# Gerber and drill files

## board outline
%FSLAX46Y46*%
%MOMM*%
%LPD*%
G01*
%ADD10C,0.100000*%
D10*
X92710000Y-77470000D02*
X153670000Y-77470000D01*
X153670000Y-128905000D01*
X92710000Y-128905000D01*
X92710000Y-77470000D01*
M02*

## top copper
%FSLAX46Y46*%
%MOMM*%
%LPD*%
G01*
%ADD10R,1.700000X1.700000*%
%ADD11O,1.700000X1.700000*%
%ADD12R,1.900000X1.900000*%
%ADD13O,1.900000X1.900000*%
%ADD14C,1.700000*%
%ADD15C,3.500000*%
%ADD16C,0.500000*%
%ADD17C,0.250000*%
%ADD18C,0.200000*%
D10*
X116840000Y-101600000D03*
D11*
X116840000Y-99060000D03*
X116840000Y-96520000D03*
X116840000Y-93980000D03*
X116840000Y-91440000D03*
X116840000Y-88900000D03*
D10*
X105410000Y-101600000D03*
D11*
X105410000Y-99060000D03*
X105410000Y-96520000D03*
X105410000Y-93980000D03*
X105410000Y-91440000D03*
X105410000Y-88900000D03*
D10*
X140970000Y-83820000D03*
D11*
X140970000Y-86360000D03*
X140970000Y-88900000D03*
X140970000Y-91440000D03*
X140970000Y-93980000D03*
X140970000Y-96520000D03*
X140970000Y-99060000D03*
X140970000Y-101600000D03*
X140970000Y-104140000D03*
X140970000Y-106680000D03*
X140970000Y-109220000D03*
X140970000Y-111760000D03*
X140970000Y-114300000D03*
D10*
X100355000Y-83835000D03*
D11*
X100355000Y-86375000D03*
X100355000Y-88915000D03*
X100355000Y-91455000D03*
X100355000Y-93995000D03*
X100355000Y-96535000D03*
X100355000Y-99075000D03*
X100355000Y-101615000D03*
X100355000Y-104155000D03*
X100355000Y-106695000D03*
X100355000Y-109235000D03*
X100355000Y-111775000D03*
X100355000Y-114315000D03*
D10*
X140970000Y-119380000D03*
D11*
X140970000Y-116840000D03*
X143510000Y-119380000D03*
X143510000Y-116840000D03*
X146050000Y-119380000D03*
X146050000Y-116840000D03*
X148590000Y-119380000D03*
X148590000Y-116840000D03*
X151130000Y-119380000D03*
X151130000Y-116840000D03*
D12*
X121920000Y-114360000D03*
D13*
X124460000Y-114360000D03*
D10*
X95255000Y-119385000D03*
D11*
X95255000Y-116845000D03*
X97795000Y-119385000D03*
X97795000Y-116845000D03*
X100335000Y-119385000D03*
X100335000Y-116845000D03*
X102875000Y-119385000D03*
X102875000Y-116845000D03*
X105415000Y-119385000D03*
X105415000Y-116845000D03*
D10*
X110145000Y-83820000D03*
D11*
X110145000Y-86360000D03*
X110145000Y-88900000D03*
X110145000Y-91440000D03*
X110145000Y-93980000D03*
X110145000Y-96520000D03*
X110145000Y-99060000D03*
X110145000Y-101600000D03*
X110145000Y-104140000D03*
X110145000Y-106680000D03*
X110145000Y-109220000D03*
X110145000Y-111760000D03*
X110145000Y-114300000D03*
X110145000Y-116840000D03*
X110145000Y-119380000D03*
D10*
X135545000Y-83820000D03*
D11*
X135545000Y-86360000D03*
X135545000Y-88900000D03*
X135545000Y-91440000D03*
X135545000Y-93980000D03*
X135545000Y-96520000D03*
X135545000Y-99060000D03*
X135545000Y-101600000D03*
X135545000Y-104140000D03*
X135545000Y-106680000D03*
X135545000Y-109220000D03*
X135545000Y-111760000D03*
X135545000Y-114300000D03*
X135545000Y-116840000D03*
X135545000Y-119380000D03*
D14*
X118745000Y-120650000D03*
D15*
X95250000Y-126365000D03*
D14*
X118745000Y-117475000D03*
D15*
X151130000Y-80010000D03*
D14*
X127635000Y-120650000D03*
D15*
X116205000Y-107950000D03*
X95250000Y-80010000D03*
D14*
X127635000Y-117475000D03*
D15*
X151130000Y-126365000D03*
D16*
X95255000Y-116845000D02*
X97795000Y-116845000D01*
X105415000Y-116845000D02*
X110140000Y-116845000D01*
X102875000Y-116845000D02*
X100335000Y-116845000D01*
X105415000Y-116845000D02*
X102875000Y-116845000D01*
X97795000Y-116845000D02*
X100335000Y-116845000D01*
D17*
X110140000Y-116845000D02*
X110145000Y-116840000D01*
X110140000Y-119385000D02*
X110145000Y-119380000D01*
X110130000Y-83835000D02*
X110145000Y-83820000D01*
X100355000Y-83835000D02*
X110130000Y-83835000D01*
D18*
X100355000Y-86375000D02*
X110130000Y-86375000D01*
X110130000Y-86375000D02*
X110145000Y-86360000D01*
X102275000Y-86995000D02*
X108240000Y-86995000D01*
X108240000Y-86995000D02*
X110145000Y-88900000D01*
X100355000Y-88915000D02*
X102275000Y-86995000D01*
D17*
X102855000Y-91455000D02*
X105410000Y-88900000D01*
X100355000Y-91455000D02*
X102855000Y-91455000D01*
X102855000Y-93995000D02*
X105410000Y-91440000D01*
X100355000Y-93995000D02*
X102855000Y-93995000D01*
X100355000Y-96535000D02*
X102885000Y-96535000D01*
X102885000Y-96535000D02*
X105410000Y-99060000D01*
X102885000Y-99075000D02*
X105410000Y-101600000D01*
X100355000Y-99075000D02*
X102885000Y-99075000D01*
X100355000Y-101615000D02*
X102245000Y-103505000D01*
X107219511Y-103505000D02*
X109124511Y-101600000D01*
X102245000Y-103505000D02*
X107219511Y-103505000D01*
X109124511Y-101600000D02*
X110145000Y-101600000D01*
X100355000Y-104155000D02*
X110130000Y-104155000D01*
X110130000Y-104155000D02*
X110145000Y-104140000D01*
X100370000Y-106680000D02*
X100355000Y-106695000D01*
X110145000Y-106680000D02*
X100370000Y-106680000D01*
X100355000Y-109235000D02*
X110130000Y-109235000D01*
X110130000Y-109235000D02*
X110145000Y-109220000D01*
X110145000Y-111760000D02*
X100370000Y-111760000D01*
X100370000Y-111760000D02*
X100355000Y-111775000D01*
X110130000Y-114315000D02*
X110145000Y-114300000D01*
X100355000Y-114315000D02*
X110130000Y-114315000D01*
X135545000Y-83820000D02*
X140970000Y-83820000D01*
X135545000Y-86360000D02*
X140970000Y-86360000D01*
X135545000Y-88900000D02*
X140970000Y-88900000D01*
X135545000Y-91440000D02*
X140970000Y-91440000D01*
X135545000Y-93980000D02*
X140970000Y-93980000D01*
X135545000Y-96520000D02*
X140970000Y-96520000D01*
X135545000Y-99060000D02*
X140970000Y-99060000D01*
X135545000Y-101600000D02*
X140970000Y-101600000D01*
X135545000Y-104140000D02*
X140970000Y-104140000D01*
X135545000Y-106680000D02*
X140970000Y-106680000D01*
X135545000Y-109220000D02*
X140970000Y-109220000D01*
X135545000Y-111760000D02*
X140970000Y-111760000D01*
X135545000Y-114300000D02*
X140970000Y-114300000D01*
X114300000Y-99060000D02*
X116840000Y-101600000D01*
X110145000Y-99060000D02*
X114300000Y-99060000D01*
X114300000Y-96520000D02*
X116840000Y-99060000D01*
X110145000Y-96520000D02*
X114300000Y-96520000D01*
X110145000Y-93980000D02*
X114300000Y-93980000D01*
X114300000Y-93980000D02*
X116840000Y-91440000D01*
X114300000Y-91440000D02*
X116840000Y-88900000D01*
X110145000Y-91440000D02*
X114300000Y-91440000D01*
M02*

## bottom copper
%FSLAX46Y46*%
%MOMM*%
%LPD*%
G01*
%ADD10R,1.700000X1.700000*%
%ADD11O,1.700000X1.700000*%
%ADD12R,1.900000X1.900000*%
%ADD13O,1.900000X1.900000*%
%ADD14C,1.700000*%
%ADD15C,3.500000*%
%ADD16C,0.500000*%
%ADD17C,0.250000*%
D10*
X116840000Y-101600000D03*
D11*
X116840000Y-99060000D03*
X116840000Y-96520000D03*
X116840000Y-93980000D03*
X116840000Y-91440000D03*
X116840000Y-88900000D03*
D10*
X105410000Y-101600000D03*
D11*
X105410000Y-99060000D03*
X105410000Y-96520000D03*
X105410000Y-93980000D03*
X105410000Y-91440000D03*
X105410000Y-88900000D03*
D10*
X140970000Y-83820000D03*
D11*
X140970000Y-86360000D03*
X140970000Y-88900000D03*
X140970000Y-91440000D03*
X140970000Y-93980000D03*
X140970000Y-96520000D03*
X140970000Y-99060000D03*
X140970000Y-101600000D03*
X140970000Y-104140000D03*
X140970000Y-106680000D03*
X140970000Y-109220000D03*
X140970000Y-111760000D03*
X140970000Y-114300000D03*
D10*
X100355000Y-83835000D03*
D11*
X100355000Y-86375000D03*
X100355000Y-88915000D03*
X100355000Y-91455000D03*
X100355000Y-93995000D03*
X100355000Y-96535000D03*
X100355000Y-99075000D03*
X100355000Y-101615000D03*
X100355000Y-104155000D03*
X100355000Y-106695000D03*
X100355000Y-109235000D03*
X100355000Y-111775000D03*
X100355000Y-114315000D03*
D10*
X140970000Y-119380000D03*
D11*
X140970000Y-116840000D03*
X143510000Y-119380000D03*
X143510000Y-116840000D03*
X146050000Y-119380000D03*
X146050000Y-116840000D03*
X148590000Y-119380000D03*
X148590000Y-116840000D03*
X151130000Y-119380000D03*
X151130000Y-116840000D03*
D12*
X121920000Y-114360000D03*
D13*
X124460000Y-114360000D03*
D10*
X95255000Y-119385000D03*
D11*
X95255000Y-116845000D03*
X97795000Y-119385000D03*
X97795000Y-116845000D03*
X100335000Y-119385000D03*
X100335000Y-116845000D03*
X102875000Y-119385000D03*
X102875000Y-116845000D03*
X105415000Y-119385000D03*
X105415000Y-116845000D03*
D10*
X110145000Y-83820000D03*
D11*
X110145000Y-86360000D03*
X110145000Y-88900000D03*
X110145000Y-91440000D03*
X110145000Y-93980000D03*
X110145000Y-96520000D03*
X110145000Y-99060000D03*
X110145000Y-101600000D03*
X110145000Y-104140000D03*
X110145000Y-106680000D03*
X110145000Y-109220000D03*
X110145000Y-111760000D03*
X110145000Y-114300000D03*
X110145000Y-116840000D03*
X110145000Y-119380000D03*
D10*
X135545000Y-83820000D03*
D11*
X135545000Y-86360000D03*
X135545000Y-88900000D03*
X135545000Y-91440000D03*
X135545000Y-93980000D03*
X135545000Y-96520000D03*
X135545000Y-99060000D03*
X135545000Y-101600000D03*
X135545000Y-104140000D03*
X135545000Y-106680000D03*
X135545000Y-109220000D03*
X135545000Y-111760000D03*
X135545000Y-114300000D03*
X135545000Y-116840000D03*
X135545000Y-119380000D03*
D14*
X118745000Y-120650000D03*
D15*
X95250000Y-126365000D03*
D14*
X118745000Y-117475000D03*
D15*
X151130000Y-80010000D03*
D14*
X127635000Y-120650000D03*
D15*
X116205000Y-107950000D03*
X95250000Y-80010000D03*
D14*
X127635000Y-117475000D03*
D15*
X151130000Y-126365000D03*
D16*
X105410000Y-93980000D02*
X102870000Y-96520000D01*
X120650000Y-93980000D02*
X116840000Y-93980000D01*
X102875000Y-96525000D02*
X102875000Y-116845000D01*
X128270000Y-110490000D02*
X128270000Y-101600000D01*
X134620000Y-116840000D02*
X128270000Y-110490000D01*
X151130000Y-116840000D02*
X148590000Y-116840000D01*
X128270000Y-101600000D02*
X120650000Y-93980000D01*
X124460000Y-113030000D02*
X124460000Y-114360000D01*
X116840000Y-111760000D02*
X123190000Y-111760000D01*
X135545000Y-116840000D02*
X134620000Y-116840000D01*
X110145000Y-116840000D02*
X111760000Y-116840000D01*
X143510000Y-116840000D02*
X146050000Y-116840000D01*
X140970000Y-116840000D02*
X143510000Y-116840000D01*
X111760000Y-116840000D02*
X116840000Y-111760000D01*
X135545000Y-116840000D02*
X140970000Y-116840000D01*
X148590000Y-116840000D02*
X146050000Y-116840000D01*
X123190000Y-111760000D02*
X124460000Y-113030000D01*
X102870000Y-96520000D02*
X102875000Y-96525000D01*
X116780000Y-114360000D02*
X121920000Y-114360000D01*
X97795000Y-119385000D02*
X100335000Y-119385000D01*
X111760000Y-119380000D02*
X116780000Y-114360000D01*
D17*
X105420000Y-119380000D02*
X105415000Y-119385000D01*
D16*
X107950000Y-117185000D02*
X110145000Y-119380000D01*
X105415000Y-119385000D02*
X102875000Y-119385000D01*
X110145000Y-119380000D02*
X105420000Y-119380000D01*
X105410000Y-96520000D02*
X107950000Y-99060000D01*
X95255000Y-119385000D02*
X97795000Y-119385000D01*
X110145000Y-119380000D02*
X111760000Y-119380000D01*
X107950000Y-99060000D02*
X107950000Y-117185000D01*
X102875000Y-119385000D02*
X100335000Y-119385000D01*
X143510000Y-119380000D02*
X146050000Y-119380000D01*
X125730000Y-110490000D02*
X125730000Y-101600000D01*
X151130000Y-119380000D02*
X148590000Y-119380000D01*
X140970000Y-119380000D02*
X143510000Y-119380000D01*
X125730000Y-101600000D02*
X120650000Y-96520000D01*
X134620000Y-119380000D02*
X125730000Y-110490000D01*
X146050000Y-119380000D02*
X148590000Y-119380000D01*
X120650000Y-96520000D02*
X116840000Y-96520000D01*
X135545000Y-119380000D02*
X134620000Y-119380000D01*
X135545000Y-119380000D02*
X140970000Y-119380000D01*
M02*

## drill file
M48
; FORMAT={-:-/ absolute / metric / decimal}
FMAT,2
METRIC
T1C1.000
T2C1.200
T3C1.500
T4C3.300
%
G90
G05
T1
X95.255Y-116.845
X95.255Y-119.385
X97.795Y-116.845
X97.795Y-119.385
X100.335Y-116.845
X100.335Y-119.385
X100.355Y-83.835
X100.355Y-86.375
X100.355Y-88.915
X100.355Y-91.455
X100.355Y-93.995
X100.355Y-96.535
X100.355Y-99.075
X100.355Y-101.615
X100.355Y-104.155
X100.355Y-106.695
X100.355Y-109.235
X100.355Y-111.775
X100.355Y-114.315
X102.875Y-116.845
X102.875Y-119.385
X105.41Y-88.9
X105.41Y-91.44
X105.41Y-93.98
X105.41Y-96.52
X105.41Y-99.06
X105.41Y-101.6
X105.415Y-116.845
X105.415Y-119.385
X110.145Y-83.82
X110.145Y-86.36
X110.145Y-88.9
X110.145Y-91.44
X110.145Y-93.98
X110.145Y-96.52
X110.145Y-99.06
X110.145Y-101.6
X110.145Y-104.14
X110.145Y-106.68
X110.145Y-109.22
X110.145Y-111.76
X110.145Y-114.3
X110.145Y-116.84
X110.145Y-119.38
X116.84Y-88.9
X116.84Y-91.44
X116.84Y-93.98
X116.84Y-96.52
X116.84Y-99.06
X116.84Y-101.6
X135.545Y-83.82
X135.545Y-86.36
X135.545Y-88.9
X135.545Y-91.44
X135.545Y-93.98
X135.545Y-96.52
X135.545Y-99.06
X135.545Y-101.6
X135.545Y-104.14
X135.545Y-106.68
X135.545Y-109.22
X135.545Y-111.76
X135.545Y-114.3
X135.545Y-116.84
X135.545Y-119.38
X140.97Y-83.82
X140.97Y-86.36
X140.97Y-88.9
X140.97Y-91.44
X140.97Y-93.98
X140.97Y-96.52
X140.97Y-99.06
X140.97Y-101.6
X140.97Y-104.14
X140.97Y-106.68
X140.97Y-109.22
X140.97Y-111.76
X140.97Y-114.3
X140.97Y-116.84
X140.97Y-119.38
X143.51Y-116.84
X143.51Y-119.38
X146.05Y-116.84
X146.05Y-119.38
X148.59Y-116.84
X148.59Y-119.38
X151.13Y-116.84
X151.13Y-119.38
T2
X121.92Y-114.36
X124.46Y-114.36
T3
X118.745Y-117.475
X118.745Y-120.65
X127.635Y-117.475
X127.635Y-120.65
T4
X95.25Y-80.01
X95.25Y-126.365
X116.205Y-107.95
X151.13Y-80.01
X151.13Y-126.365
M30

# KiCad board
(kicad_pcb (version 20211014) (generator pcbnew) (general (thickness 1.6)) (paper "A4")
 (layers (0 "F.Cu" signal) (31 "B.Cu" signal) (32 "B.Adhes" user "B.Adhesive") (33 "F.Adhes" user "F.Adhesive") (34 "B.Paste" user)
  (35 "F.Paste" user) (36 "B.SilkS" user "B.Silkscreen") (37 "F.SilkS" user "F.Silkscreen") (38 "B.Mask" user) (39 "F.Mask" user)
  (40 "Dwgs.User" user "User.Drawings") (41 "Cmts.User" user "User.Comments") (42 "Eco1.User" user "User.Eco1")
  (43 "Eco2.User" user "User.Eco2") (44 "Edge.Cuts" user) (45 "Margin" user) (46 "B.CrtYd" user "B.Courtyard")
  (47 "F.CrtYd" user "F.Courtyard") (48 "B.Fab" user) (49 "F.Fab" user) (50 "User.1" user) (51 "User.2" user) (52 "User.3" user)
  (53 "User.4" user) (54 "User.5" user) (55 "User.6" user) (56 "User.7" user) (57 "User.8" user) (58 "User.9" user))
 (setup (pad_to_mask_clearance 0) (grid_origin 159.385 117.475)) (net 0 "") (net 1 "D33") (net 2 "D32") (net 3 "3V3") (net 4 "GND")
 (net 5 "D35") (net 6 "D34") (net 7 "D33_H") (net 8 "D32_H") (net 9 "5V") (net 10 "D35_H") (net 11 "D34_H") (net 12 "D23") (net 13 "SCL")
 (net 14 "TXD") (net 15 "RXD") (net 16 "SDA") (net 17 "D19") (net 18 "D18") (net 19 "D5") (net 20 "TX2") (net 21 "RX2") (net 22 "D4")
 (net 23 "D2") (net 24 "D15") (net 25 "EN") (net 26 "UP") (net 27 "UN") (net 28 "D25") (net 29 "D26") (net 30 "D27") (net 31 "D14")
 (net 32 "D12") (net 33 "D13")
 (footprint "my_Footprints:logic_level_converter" (layer "F.Cu") (at 118.11 101.6 180)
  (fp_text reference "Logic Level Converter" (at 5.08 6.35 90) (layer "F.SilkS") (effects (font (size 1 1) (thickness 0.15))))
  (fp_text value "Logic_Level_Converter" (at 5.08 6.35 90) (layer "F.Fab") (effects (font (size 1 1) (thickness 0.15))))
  (pad "1" thru_hole rect (at 1.27 0 180) (size 1.7 1.7) (drill 1) (layers *.Cu *.Mask) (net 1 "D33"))
  (pad "2" thru_hole oval (at 1.27 2.54 180) (size 1.7 1.7) (drill 1) (layers *.Cu *.Mask) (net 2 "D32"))
  (pad "3" thru_hole oval (at 1.27 5.08 180) (size 1.7 1.7) (drill 1) (layers *.Cu *.Mask) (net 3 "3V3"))
  (pad "4" thru_hole oval (at 1.27 7.62 180) (size 1.7 1.7) (drill 1) (layers *.Cu *.Mask) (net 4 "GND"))
  (pad "5" thru_hole oval (at 1.27 10.16 180) (size 1.7 1.7) (drill 1) (layers *.Cu *.Mask) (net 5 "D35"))
  (pad "6" thru_hole oval (at 1.27 12.7 180) (size 1.7 1.7) (drill 1) (layers *.Cu *.Mask) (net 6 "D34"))
  (pad "7" thru_hole rect (at 12.7 0 180) (size 1.7 1.7) (drill 1) (layers *.Cu *.Mask) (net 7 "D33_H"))
  (pad "8" thru_hole oval (at 12.7 2.54 180) (size 1.7 1.7) (drill 1) (layers *.Cu *.Mask) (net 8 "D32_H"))
  (pad "9" thru_hole oval (at 12.7 5.08 180) (size 1.7 1.7) (drill 1) (layers *.Cu *.Mask) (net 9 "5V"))
  (pad "10" thru_hole oval (at 12.7 7.62 180) (size 1.7 1.7) (drill 1) (layers *.Cu *.Mask) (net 4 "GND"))
  (pad "11" thru_hole oval (at 12.7 10.16 180) (size 1.7 1.7) (drill 1) (layers *.Cu *.Mask) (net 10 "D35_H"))
  (pad "12" thru_hole oval (at 12.7 12.7 180) (size 1.7 1.7) (drill 1) (layers *.Cu *.Mask) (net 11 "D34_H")))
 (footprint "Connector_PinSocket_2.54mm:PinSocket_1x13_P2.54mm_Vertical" (layer "F.Cu") (at 140.97 83.82)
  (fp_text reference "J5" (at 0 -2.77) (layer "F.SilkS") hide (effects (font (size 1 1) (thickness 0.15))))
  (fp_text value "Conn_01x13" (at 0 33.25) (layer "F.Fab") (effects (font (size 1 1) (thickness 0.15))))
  (pad "1" thru_hole rect (at 0 0) (size 1.7 1.7) (drill 1) (layers *.Cu *.Mask) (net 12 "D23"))
  (pad "2" thru_hole oval (at 0 2.54) (size 1.7 1.7) (drill 1) (layers *.Cu *.Mask) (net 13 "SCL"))
  (pad "3" thru_hole oval (at 0 5.08) (size 1.7 1.7) (drill 1) (layers *.Cu *.Mask) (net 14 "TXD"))
  (pad "4" thru_hole oval (at 0 7.62) (size 1.7 1.7) (drill 1) (layers *.Cu *.Mask) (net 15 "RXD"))
  (pad "5" thru_hole oval (at 0 10.16) (size 1.7 1.7) (drill 1) (layers *.Cu *.Mask) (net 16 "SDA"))
  (pad "6" thru_hole oval (at 0 12.7) (size 1.7 1.7) (drill 1) (layers *.Cu *.Mask) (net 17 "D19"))
  (pad "7" thru_hole oval (at 0 15.24) (size 1.7 1.7) (drill 1) (layers *.Cu *.Mask) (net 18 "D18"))
  (pad "8" thru_hole oval (at 0 17.78) (size 1.7 1.7) (drill 1) (layers *.Cu *.Mask) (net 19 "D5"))
  (pad "9" thru_hole oval (at 0 20.32) (size 1.7 1.7) (drill 1) (layers *.Cu *.Mask) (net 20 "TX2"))
  (pad "10" thru_hole oval (at 0 22.86) (size 1.7 1.7) (drill 1) (layers *.Cu *.Mask) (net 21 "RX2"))
  (pad "11" thru_hole oval (at 0 25.4) (size 1.7 1.7) (drill 1) (layers *.Cu *.Mask) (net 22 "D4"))
  (pad "12" thru_hole oval (at 0 27.94) (size 1.7 1.7) (drill 1) (layers *.Cu *.Mask) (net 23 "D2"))
  (pad "13" thru_hole oval (at 0 30.48) (size 1.7 1.7) (drill 1) (layers *.Cu *.Mask) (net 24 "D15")))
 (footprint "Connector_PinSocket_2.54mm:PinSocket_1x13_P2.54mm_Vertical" (layer "F.Cu") (at 100.355 83.835)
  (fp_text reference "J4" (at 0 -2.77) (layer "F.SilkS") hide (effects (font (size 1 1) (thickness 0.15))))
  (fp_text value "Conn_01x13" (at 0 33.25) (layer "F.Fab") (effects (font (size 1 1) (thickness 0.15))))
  (pad "1" thru_hole rect (at 0 0) (size 1.7 1.7) (drill 1) (layers *.Cu *.Mask) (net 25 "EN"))
  (pad "2" thru_hole oval (at 0 2.54) (size 1.7 1.7) (drill 1) (layers *.Cu *.Mask) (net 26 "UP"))
  (pad "3" thru_hole oval (at 0 5.08) (size 1.7 1.7) (drill 1) (layers *.Cu *.Mask) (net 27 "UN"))
  (pad "4" thru_hole oval (at 0 7.62) (size 1.7 1.7) (drill 1) (layers *.Cu *.Mask) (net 11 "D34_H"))
  (pad "5" thru_hole oval (at 0 10.16) (size 1.7 1.7) (drill 1) (layers *.Cu *.Mask) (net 10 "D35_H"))
  (pad "6" thru_hole oval (at 0 12.7) (size 1.7 1.7) (drill 1) (layers *.Cu *.Mask) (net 8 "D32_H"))
  (pad "7" thru_hole oval (at 0 15.24) (size 1.7 1.7) (drill 1) (layers *.Cu *.Mask) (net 7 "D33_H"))
  (pad "8" thru_hole oval (at 0 17.78) (size 1.7 1.7) (drill 1) (layers *.Cu *.Mask) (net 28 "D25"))
  (pad "9" thru_hole oval (at 0 20.32) (size 1.7 1.7) (drill 1) (layers *.Cu *.Mask) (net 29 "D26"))
  (pad "10" thru_hole oval (at 0 22.86) (size 1.7 1.7) (drill 1) (layers *.Cu *.Mask) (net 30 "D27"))
  (pad "11" thru_hole oval (at 0 25.4) (size 1.7 1.7) (drill 1) (layers *.Cu *.Mask) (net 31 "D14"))
  (pad "12" thru_hole oval (at 0 27.94) (size 1.7 1.7) (drill 1) (layers *.Cu *.Mask) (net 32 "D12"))
  (pad "13" thru_hole oval (at 0 30.48) (size 1.7 1.7) (drill 1) (layers *.Cu *.Mask) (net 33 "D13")))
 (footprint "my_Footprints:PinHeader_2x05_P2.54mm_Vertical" (layer "F.Cu") (at 140.97 119.38 90)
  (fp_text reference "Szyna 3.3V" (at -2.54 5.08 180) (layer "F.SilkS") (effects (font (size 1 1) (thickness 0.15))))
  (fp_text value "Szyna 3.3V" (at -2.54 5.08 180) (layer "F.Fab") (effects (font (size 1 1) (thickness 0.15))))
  (pad "1" thru_hole rect (at 0 0 90) (size 1.7 1.7) (drill 1) (layers *.Cu *.Mask) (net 3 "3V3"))
  (pad "2" thru_hole oval (at 2.54 0 90) (size 1.7 1.7) (drill 1) (layers *.Cu *.Mask) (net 4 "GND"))
  (pad "3" thru_hole oval (at 0 2.54 90) (size 1.7 1.7) (drill 1) (layers *.Cu *.Mask) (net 3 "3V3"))
  (pad "4" thru_hole oval (at 2.54 2.54 90) (size 1.7 1.7) (drill 1) (layers *.Cu *.Mask) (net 4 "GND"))
  (pad "5" thru_hole oval (at 0 5.08 90) (size 1.7 1.7) (drill 1) (layers *.Cu *.Mask) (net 3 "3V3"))
  (pad "6" thru_hole oval (at 2.54 5.08 90) (size 1.7 1.7) (drill 1) (layers *.Cu *.Mask) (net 4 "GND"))
  (pad "7" thru_hole oval (at 0 7.62 90) (size 1.7 1.7) (drill 1) (layers *.Cu *.Mask) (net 3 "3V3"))
  (pad "8" thru_hole oval (at 2.54 7.62 90) (size 1.7 1.7) (drill 1) (layers *.Cu *.Mask) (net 4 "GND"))
  (pad "9" thru_hole oval (at 0 10.16 90) (size 1.7 1.7) (drill 1) (layers *.Cu *.Mask) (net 3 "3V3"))
  (pad "10" thru_hole oval (at 2.54 10.16 90) (size 1.7 1.7) (drill 1) (layers *.Cu *.Mask) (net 4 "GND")))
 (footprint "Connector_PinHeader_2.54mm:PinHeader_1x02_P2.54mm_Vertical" (layer "F.Cu") (at 121.92 114.36 90)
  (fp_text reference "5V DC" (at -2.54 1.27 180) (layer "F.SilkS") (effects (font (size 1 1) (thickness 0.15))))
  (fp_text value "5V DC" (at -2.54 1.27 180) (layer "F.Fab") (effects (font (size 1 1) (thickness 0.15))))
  (pad "1" thru_hole rect (at 0 0 90) (size 1.9 1.9) (drill 1.2) (layers *.Cu *.Mask) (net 9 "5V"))
  (pad "2" thru_hole oval (at 0 2.54 90) (size 1.9 1.9) (drill 1.2) (layers *.Cu *.Mask) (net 4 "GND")))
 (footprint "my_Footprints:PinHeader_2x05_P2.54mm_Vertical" (layer "F.Cu") (at 95.255 119.385 90)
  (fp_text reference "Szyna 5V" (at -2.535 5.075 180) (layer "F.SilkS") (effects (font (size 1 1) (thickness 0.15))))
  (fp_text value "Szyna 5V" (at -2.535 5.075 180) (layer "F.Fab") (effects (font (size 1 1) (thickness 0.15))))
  (pad "1" thru_hole rect (at 0 0 90) (size 1.7 1.7) (drill 1) (layers *.Cu *.Mask) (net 9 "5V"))
  (pad "2" thru_hole oval (at 2.54 0 90) (size 1.7 1.7) (drill 1) (layers *.Cu *.Mask) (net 4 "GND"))
  (pad "3" thru_hole oval (at 0 2.54 90) (size 1.7 1.7) (drill 1) (layers *.Cu *.Mask) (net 9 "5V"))
  (pad "4" thru_hole oval (at 2.54 2.54 90) (size 1.7 1.7) (drill 1) (layers *.Cu *.Mask) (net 4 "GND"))
  (pad "5" thru_hole oval (at 0 5.08 90) (size 1.7 1.7) (drill 1) (layers *.Cu *.Mask) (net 9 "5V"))
  (pad "6" thru_hole oval (at 2.54 5.08 90) (size 1.7 1.7) (drill 1) (layers *.Cu *.Mask) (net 4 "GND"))
  (pad "7" thru_hole oval (at 0 7.62 90) (size 1.7 1.7) (drill 1) (layers *.Cu *.Mask) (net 9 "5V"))
  (pad "8" thru_hole oval (at 2.54 7.62 90) (size 1.7 1.7) (drill 1) (layers *.Cu *.Mask) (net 4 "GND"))
  (pad "9" thru_hole oval (at 0 10.16 90) (size 1.7 1.7) (drill 1) (layers *.Cu *.Mask) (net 9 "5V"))
  (pad "10" thru_hole oval (at 2.54 10.16 90) (size 1.7 1.7) (drill 1) (layers *.Cu *.Mask) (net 4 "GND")))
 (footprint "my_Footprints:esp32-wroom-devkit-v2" (layer "F.Cu") (at 110.145 83.82)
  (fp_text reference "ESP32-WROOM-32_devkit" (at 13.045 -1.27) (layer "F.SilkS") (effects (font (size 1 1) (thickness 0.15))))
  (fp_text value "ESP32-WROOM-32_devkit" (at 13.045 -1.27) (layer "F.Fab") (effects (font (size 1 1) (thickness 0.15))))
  (pad "1" thru_hole rect (at 0 0) (size 1.7 1.7) (drill 1) (layers *.Cu *.Mask) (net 25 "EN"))
  (pad "2" thru_hole oval (at 0 2.54) (size 1.7 1.7) (drill 1) (layers *.Cu *.Mask) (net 26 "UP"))
  (pad "3" thru_hole oval (at 0 5.08) (size 1.7 1.7) (drill 1) (layers *.Cu *.Mask) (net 27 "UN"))
  (pad "4" thru_hole oval (at 0 7.62) (size 1.7 1.7) (drill 1) (layers *.Cu *.Mask) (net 6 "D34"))
  (pad "5" thru_hole oval (at 0 10.16) (size 1.7 1.7) (drill 1) (layers *.Cu *.Mask) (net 5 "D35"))
  (pad "6" thru_hole oval (at 0 12.7) (size 1.7 1.7) (drill 1) (layers *.Cu *.Mask) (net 2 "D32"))
  (pad "7" thru_hole oval (at 0 15.24) (size 1.7 1.7) (drill 1) (layers *.Cu *.Mask) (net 1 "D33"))
  (pad "8" thru_hole oval (at 0 17.78) (size 1.7 1.7) (drill 1) (layers *.Cu *.Mask) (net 28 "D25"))
  (pad "9" thru_hole oval (at 0 20.32) (size 1.7 1.7) (drill 1) (layers *.Cu *.Mask) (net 29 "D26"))
  (pad "10" thru_hole oval (at 0 22.86) (size 1.7 1.7) (drill 1) (layers *.Cu *.Mask) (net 30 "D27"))
  (pad "11" thru_hole oval (at 0 25.4) (size 1.7 1.7) (drill 1) (layers *.Cu *.Mask) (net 31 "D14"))
  (pad "12" thru_hole oval (at 0 27.94) (size 1.7 1.7) (drill 1) (layers *.Cu *.Mask) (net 32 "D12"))
  (pad "13" thru_hole oval (at 0 30.48) (size 1.7 1.7) (drill 1) (layers *.Cu *.Mask) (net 33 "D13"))
  (pad "14" thru_hole oval (at 0 33.02) (size 1.7 1.7) (drill 1) (layers *.Cu *.Mask) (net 4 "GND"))
  (pad "15" thru_hole oval (at 0 35.56) (size 1.7 1.7) (drill 1) (layers *.Cu *.Mask) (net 9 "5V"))
  (pad "16" thru_hole rect (at 25.4 0) (size 1.7 1.7) (drill 1) (layers *.Cu *.Mask) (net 12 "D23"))
  (pad "17" thru_hole oval (at 25.4 2.54) (size 1.7 1.7) (drill 1) (layers *.Cu *.Mask) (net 13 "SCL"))
  (pad "18" thru_hole oval (at 25.4 5.08) (size 1.7 1.7) (drill 1) (layers *.Cu *.Mask) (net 14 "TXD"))
  (pad "19" thru_hole oval (at 25.4 7.62) (size 1.7 1.7) (drill 1) (layers *.Cu *.Mask) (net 15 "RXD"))
  (pad "20" thru_hole oval (at 25.4 10.16) (size 1.7 1.7) (drill 1) (layers *.Cu *.Mask) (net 16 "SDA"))
  (pad "21" thru_hole oval (at 25.4 12.7) (size 1.7 1.7) (drill 1) (layers *.Cu *.Mask) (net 17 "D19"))
  (pad "22" thru_hole oval (at 25.4 15.24) (size 1.7 1.7) (drill 1) (layers *.Cu *.Mask) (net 18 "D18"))
  (pad "23" thru_hole oval (at 25.4 17.78) (size 1.7 1.7) (drill 1) (layers *.Cu *.Mask) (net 19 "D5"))
  (pad "24" thru_hole oval (at 25.4 20.32) (size 1.7 1.7) (drill 1) (layers *.Cu *.Mask) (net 20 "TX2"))
  (pad "25" thru_hole oval (at 25.4 22.86) (size 1.7 1.7) (drill 1) (layers *.Cu *.Mask) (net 21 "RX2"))
  (pad "26" thru_hole oval (at 25.4 25.4) (size 1.7 1.7) (drill 1) (layers *.Cu *.Mask) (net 22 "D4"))
  (pad "27" thru_hole oval (at 25.4 27.94) (size 1.7 1.7) (drill 1) (layers *.Cu *.Mask) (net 23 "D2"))
  (pad "28" thru_hole oval (at 25.4 30.48) (size 1.7 1.7) (drill 1) (layers *.Cu *.Mask) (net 24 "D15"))
  (pad "29" thru_hole oval (at 25.4 33.02) (size 1.7 1.7) (drill 1) (layers *.Cu *.Mask) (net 4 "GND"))
  (pad "30" thru_hole oval (at 25.4 35.56) (size 1.7 1.7) (drill 1) (layers *.Cu *.Mask) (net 3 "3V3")))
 (gr_rect (start 92.71 77.47) (end 153.67 128.905) (layer "Edge.Cuts") (width 0.1) (fill none))
 (via (at 118.745 120.65) (size 1.7) (drill 1.5) (layers "F.Cu" "B.Cu") (free) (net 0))
 (via (at 95.25 126.365) (size 3.5) (drill 3.3) (layers "F.Cu" "B.Cu") (free) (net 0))
 (via (at 118.745 117.475) (size 1.7) (drill 1.5) (layers "F.Cu" "B.Cu") (free) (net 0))
 (via (at 151.13 80.01) (size 3.5) (drill 3.3) (layers "F.Cu" "B.Cu") (free) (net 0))
 (via (at 127.635 120.65) (size 1.7) (drill 1.5) (layers "F.Cu" "B.Cu") (free) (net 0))
 (via (at 116.205 107.95) (size 3.5) (drill 3.3) (layers "F.Cu" "B.Cu") (free) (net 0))
 (via (at 95.25 80.01) (size 3.5) (drill 3.3) (layers "F.Cu" "B.Cu") (free) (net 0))
 (via (at 127.635 117.475) (size 1.7) (drill 1.5) (layers "F.Cu" "B.Cu") (free) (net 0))
 (via (at 151.13 126.365) (size 3.5) (drill 3.3) (layers "F.Cu" "B.Cu") (free) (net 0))
 (segment (start 95.255 116.845) (end 97.795 116.845) (width 0.5) (layer "F.Cu") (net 4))
 (segment (start 105.415 116.845) (end 110.14 116.845) (width 0.5) (layer "F.Cu") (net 4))
 (segment (start 102.875 116.845) (end 100.335 116.845) (width 0.5) (layer "F.Cu") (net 4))
 (segment (start 105.415 116.845) (end 102.875 116.845) (width 0.5) (layer "F.Cu") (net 4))
 (segment (start 97.795 116.845) (end 100.335 116.845) (width 0.5) (layer "F.Cu") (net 4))
 (segment (start 110.14 116.845) (end 110.145 116.84) (width 0.25) (layer "F.Cu") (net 4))
 (segment (start 105.41 93.98) (end 102.87 96.52) (width 0.5) (layer "B.Cu") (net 4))
 (segment (start 120.65 93.98) (end 116.84 93.98) (width 0.5) (layer "B.Cu") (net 4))
 (segment (start 102.875 96.525) (end 102.875 116.845) (width 0.5) (layer "B.Cu") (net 4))
 (segment (start 128.27 110.49) (end 128.27 101.6) (width 0.5) (layer "B.Cu") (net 4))
 (segment (start 134.62 116.84) (end 128.27 110.49) (width 0.5) (layer "B.Cu") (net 4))
 (segment (start 151.13 116.84) (end 148.59 116.84) (width 0.5) (layer "B.Cu") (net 4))
 (segment (start 128.27 101.6) (end 120.65 93.98) (width 0.5) (layer "B.Cu") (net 4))
 (segment (start 124.46 113.03) (end 124.46 114.36) (width 0.5) (layer "B.Cu") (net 4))
 (segment (start 116.84 111.76) (end 123.19 111.76) (width 0.5) (layer "B.Cu") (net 4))
 (segment (start 135.545 116.84) (end 134.62 116.84) (width 0.5) (layer "B.Cu") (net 4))
 (segment (start 110.145 116.84) (end 111.76 116.84) (width 0.5) (layer "B.Cu") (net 4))
 (segment (start 143.51 116.84) (end 146.05 116.84) (width 0.5) (layer "B.Cu") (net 4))
 (segment (start 140.97 116.84) (end 143.51 116.84) (width 0.5) (layer "B.Cu") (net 4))
 (segment (start 111.76 116.84) (end 116.84 111.76) (width 0.5) (layer "B.Cu") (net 4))
 (segment (start 135.545 116.84) (end 140.97 116.84) (width 0.5) (layer "B.Cu") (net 4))
 (segment (start 148.59 116.84) (end 146.05 116.84) (width 0.5) (layer "B.Cu") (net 4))
 (segment (start 123.19 111.76) (end 124.46 113.03) (width 0.5) (layer "B.Cu") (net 4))
 (segment (start 102.87 96.52) (end 102.875 96.525) (width 0.5) (layer "B.Cu") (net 4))
 (segment (start 110.14 119.385) (end 110.145 119.38) (width 0.25) (layer "F.Cu") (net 9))
 (segment (start 116.78 114.36) (end 121.92 114.36) (width 0.5) (layer "B.Cu") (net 9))
 (segment (start 97.795 119.385) (end 100.335 119.385) (width 0.5) (layer "B.Cu") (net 9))
 (segment (start 111.76 119.38) (end 116.78 114.36) (width 0.5) (layer "B.Cu") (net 9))
 (segment (start 105.42 119.38) (end 105.415 119.385) (width 0.25) (layer "B.Cu") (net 9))
 (segment (start 107.95 117.185) (end 110.145 119.38) (width 0.5) (layer "B.Cu") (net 9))
 (segment (start 105.415 119.385) (end 102.875 119.385) (width 0.5) (layer "B.Cu") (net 9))
 (segment (start 110.145 119.38) (end 105.42 119.38) (width 0.5) (layer "B.Cu") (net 9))
 (segment (start 105.41 96.52) (end 107.95 99.06) (width 0.5) (layer "B.Cu") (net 9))
 (segment (start 95.255 119.385) (end 97.795 119.385) (width 0.5) (layer "B.Cu") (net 9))
 (segment (start 110.145 119.38) (end 111.76 119.38) (width 0.5) (layer "B.Cu") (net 9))
 (segment (start 107.95 99.06) (end 107.95 117.185) (width 0.5) (layer "B.Cu") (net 9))
 (segment (start 102.875 119.385) (end 100.335 119.385) (width 0.5) (layer "B.Cu") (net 9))
 (segment (start 110.13 83.835) (end 110.145 83.82) (width 0.25) (layer "F.Cu") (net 25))
 (segment (start 100.355 83.835) (end 110.13 83.835) (width 0.25) (layer "F.Cu") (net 25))
 (segment (start 100.355 86.375) (end 110.13 86.375) (width 0.2) (layer "F.Cu") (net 26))
 (segment (start 110.13 86.375) (end 110.145 86.36) (width 0.2) (layer "F.Cu") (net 26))
 (segment (start 102.275 86.995) (end 108.24 86.995) (width 0.2) (layer "F.Cu") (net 27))
 (segment (start 108.24 86.995) (end 110.145 88.9) (width 0.2) (layer "F.Cu") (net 27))
 (segment (start 100.355 88.915) (end 102.275 86.995) (width 0.2) (layer "F.Cu") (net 27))
 (segment (start 102.855 91.455) (end 105.41 88.9) (width 0.25) (layer "F.Cu") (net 11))
 (segment (start 100.355 91.455) (end 102.855 91.455) (width 0.25) (layer "F.Cu") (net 11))
 (segment (start 102.855 93.995) (end 105.41 91.44) (width 0.25) (layer "F.Cu") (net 10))
 (segment (start 100.355 93.995) (end 102.855 93.995) (width 0.25) (layer "F.Cu") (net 10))
 (segment (start 100.355 96.535) (end 102.885 96.535) (width 0.25) (layer "F.Cu") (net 8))
 (segment (start 102.885 96.535) (end 105.41 99.06) (width 0.25) (layer "F.Cu") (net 8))
 (segment (start 102.885 99.075) (end 105.41 101.6) (width 0.25) (layer "F.Cu") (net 7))
 (segment (start 100.355 99.075) (end 102.885 99.075) (width 0.25) (layer "F.Cu") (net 7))
 (segment (start 100.355 101.615) (end 102.245 103.505) (width 0.25) (layer "F.Cu") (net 28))
 (segment (start 107.219511 103.505) (end 109.124511 101.6) (width 0.25) (layer "F.Cu") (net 28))
 (segment (start 102.245 103.505) (end 107.219511 103.505) (width 0.25) (layer "F.Cu") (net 28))
 (segment (start 109.124511 101.6) (end 110.145 101.6) (width 0.25) (layer "F.Cu") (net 28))
 (segment (start 100.355 104.155) (end 110.13 104.155) (width 0.25) (layer "F.Cu") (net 29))
 (segment (start 110.13 104.155) (end 110.145 104.14) (width 0.25) (layer "F.Cu") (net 29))
 (segment (start 100.37 106.68) (end 100.355 106.695) (width 0.25) (layer "F.Cu") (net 30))
 (segment (start 110.145 106.68) (end 100.37 106.68) (width 0.25) (layer "F.Cu") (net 30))
 (segment (start 100.355 109.235) (end 110.13 109.235) (width 0.25) (layer "F.Cu") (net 31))
 (segment (start 110.13 109.235) (end 110.145 109.22) (width 0.25) (layer "F.Cu") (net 31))
 (segment (start 110.145 111.76) (end 100.37 111.76) (width 0.25) (layer "F.Cu") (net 32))
 (segment (start 100.37 111.76) (end 100.355 111.775) (width 0.25) (layer "F.Cu") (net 32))
 (segment (start 110.13 114.315) (end 110.145 114.3) (width 0.25) (layer "F.Cu") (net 33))
 (segment (start 100.355 114.315) (end 110.13 114.315) (width 0.25) (layer "F.Cu") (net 33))
 (segment (start 135.545 83.82) (end 140.97 83.82) (width 0.25) (layer "F.Cu") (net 12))
 (segment (start 135.545 86.36) (end 140.97 86.36) (width 0.25) (layer "F.Cu") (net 13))
 (segment (start 135.545 88.9) (end 140.97 88.9) (width 0.25) (layer "F.Cu") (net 14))
 (segment (start 135.545 91.44) (end 140.97 91.44) (width 0.25) (layer "F.Cu") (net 15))
 (segment (start 135.545 93.98) (end 140.97 93.98) (width 0.25) (layer "F.Cu") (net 16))
 (segment (start 135.545 96.52) (end 140.97 96.52) (width 0.25) (layer "F.Cu") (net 17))
 (segment (start 135.545 99.06) (end 140.97 99.06) (width 0.25) (layer "F.Cu") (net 18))
 (segment (start 135.545 101.6) (end 140.97 101.6) (width 0.25) (layer "F.Cu") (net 19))
 (segment (start 135.545 104.14) (end 140.97 104.14) (width 0.25) (layer "F.Cu") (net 20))
 (segment (start 135.545 106.68) (end 140.97 106.68) (width 0.25) (layer "F.Cu") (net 21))
 (segment (start 135.545 109.22) (end 140.97 109.22) (width 0.25) (layer "F.Cu") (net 22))
 (segment (start 135.545 111.76) (end 140.97 111.76) (width 0.25) (layer "F.Cu") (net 23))
 (segment (start 135.545 114.3) (end 140.97 114.3) (width 0.25) (layer "F.Cu") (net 24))
 (segment (start 143.51 119.38) (end 146.05 119.38) (width 0.5) (layer "B.Cu") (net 3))
 (segment (start 125.73 110.49) (end 125.73 101.6) (width 0.5) (layer "B.Cu") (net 3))
 (segment (start 151.13 119.38) (end 148.59 119.38) (width 0.5) (layer "B.Cu") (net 3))
 (segment (start 140.97 119.38) (end 143.51 119.38) (width 0.5) (layer "B.Cu") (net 3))
 (segment (start 125.73 101.6) (end 120.65 96.52) (width 0.5) (layer "B.Cu") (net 3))
 (segment (start 134.62 119.38) (end 125.73 110.49) (width 0.5) (layer "B.Cu") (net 3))
 (segment (start 146.05 119.38) (end 148.59 119.38) (width 0.5) (layer "B.Cu") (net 3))
 (segment (start 120.65 96.52) (end 116.84 96.52) (width 0.5) (layer "B.Cu") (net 3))
 (segment (start 135.545 119.38) (end 134.62 119.38) (width 0.5) (layer "B.Cu") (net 3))
 (segment (start 135.545 119.38) (end 140.97 119.38) (width 0.5) (layer "B.Cu") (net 3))
 (segment (start 114.3 99.06) (end 116.84 101.6) (width 0.25) (layer "F.Cu") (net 1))
 (segment (start 110.145 99.06) (end 114.3 99.06) (width 0.25) (layer "F.Cu") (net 1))
 (segment (start 114.3 96.52) (end 116.84 99.06) (width 0.25) (layer "F.Cu") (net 2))
 (segment (start 110.145 96.52) (end 114.3 96.52) (width 0.25) (layer "F.Cu") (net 2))
 (segment (start 110.145 93.98) (end 114.3 93.98) (width 0.25) (layer "F.Cu") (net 5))
 (segment (start 114.3 93.98) (end 116.84 91.44) (width 0.25) (layer "F.Cu") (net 5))
 (segment (start 114.3 91.44) (end 116.84 88.9) (width 0.25) (layer "F.Cu") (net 6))
 (segment (start 110.145 91.44) (end 114.3 91.44) (width 0.25) (layer "F.Cu") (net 6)))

